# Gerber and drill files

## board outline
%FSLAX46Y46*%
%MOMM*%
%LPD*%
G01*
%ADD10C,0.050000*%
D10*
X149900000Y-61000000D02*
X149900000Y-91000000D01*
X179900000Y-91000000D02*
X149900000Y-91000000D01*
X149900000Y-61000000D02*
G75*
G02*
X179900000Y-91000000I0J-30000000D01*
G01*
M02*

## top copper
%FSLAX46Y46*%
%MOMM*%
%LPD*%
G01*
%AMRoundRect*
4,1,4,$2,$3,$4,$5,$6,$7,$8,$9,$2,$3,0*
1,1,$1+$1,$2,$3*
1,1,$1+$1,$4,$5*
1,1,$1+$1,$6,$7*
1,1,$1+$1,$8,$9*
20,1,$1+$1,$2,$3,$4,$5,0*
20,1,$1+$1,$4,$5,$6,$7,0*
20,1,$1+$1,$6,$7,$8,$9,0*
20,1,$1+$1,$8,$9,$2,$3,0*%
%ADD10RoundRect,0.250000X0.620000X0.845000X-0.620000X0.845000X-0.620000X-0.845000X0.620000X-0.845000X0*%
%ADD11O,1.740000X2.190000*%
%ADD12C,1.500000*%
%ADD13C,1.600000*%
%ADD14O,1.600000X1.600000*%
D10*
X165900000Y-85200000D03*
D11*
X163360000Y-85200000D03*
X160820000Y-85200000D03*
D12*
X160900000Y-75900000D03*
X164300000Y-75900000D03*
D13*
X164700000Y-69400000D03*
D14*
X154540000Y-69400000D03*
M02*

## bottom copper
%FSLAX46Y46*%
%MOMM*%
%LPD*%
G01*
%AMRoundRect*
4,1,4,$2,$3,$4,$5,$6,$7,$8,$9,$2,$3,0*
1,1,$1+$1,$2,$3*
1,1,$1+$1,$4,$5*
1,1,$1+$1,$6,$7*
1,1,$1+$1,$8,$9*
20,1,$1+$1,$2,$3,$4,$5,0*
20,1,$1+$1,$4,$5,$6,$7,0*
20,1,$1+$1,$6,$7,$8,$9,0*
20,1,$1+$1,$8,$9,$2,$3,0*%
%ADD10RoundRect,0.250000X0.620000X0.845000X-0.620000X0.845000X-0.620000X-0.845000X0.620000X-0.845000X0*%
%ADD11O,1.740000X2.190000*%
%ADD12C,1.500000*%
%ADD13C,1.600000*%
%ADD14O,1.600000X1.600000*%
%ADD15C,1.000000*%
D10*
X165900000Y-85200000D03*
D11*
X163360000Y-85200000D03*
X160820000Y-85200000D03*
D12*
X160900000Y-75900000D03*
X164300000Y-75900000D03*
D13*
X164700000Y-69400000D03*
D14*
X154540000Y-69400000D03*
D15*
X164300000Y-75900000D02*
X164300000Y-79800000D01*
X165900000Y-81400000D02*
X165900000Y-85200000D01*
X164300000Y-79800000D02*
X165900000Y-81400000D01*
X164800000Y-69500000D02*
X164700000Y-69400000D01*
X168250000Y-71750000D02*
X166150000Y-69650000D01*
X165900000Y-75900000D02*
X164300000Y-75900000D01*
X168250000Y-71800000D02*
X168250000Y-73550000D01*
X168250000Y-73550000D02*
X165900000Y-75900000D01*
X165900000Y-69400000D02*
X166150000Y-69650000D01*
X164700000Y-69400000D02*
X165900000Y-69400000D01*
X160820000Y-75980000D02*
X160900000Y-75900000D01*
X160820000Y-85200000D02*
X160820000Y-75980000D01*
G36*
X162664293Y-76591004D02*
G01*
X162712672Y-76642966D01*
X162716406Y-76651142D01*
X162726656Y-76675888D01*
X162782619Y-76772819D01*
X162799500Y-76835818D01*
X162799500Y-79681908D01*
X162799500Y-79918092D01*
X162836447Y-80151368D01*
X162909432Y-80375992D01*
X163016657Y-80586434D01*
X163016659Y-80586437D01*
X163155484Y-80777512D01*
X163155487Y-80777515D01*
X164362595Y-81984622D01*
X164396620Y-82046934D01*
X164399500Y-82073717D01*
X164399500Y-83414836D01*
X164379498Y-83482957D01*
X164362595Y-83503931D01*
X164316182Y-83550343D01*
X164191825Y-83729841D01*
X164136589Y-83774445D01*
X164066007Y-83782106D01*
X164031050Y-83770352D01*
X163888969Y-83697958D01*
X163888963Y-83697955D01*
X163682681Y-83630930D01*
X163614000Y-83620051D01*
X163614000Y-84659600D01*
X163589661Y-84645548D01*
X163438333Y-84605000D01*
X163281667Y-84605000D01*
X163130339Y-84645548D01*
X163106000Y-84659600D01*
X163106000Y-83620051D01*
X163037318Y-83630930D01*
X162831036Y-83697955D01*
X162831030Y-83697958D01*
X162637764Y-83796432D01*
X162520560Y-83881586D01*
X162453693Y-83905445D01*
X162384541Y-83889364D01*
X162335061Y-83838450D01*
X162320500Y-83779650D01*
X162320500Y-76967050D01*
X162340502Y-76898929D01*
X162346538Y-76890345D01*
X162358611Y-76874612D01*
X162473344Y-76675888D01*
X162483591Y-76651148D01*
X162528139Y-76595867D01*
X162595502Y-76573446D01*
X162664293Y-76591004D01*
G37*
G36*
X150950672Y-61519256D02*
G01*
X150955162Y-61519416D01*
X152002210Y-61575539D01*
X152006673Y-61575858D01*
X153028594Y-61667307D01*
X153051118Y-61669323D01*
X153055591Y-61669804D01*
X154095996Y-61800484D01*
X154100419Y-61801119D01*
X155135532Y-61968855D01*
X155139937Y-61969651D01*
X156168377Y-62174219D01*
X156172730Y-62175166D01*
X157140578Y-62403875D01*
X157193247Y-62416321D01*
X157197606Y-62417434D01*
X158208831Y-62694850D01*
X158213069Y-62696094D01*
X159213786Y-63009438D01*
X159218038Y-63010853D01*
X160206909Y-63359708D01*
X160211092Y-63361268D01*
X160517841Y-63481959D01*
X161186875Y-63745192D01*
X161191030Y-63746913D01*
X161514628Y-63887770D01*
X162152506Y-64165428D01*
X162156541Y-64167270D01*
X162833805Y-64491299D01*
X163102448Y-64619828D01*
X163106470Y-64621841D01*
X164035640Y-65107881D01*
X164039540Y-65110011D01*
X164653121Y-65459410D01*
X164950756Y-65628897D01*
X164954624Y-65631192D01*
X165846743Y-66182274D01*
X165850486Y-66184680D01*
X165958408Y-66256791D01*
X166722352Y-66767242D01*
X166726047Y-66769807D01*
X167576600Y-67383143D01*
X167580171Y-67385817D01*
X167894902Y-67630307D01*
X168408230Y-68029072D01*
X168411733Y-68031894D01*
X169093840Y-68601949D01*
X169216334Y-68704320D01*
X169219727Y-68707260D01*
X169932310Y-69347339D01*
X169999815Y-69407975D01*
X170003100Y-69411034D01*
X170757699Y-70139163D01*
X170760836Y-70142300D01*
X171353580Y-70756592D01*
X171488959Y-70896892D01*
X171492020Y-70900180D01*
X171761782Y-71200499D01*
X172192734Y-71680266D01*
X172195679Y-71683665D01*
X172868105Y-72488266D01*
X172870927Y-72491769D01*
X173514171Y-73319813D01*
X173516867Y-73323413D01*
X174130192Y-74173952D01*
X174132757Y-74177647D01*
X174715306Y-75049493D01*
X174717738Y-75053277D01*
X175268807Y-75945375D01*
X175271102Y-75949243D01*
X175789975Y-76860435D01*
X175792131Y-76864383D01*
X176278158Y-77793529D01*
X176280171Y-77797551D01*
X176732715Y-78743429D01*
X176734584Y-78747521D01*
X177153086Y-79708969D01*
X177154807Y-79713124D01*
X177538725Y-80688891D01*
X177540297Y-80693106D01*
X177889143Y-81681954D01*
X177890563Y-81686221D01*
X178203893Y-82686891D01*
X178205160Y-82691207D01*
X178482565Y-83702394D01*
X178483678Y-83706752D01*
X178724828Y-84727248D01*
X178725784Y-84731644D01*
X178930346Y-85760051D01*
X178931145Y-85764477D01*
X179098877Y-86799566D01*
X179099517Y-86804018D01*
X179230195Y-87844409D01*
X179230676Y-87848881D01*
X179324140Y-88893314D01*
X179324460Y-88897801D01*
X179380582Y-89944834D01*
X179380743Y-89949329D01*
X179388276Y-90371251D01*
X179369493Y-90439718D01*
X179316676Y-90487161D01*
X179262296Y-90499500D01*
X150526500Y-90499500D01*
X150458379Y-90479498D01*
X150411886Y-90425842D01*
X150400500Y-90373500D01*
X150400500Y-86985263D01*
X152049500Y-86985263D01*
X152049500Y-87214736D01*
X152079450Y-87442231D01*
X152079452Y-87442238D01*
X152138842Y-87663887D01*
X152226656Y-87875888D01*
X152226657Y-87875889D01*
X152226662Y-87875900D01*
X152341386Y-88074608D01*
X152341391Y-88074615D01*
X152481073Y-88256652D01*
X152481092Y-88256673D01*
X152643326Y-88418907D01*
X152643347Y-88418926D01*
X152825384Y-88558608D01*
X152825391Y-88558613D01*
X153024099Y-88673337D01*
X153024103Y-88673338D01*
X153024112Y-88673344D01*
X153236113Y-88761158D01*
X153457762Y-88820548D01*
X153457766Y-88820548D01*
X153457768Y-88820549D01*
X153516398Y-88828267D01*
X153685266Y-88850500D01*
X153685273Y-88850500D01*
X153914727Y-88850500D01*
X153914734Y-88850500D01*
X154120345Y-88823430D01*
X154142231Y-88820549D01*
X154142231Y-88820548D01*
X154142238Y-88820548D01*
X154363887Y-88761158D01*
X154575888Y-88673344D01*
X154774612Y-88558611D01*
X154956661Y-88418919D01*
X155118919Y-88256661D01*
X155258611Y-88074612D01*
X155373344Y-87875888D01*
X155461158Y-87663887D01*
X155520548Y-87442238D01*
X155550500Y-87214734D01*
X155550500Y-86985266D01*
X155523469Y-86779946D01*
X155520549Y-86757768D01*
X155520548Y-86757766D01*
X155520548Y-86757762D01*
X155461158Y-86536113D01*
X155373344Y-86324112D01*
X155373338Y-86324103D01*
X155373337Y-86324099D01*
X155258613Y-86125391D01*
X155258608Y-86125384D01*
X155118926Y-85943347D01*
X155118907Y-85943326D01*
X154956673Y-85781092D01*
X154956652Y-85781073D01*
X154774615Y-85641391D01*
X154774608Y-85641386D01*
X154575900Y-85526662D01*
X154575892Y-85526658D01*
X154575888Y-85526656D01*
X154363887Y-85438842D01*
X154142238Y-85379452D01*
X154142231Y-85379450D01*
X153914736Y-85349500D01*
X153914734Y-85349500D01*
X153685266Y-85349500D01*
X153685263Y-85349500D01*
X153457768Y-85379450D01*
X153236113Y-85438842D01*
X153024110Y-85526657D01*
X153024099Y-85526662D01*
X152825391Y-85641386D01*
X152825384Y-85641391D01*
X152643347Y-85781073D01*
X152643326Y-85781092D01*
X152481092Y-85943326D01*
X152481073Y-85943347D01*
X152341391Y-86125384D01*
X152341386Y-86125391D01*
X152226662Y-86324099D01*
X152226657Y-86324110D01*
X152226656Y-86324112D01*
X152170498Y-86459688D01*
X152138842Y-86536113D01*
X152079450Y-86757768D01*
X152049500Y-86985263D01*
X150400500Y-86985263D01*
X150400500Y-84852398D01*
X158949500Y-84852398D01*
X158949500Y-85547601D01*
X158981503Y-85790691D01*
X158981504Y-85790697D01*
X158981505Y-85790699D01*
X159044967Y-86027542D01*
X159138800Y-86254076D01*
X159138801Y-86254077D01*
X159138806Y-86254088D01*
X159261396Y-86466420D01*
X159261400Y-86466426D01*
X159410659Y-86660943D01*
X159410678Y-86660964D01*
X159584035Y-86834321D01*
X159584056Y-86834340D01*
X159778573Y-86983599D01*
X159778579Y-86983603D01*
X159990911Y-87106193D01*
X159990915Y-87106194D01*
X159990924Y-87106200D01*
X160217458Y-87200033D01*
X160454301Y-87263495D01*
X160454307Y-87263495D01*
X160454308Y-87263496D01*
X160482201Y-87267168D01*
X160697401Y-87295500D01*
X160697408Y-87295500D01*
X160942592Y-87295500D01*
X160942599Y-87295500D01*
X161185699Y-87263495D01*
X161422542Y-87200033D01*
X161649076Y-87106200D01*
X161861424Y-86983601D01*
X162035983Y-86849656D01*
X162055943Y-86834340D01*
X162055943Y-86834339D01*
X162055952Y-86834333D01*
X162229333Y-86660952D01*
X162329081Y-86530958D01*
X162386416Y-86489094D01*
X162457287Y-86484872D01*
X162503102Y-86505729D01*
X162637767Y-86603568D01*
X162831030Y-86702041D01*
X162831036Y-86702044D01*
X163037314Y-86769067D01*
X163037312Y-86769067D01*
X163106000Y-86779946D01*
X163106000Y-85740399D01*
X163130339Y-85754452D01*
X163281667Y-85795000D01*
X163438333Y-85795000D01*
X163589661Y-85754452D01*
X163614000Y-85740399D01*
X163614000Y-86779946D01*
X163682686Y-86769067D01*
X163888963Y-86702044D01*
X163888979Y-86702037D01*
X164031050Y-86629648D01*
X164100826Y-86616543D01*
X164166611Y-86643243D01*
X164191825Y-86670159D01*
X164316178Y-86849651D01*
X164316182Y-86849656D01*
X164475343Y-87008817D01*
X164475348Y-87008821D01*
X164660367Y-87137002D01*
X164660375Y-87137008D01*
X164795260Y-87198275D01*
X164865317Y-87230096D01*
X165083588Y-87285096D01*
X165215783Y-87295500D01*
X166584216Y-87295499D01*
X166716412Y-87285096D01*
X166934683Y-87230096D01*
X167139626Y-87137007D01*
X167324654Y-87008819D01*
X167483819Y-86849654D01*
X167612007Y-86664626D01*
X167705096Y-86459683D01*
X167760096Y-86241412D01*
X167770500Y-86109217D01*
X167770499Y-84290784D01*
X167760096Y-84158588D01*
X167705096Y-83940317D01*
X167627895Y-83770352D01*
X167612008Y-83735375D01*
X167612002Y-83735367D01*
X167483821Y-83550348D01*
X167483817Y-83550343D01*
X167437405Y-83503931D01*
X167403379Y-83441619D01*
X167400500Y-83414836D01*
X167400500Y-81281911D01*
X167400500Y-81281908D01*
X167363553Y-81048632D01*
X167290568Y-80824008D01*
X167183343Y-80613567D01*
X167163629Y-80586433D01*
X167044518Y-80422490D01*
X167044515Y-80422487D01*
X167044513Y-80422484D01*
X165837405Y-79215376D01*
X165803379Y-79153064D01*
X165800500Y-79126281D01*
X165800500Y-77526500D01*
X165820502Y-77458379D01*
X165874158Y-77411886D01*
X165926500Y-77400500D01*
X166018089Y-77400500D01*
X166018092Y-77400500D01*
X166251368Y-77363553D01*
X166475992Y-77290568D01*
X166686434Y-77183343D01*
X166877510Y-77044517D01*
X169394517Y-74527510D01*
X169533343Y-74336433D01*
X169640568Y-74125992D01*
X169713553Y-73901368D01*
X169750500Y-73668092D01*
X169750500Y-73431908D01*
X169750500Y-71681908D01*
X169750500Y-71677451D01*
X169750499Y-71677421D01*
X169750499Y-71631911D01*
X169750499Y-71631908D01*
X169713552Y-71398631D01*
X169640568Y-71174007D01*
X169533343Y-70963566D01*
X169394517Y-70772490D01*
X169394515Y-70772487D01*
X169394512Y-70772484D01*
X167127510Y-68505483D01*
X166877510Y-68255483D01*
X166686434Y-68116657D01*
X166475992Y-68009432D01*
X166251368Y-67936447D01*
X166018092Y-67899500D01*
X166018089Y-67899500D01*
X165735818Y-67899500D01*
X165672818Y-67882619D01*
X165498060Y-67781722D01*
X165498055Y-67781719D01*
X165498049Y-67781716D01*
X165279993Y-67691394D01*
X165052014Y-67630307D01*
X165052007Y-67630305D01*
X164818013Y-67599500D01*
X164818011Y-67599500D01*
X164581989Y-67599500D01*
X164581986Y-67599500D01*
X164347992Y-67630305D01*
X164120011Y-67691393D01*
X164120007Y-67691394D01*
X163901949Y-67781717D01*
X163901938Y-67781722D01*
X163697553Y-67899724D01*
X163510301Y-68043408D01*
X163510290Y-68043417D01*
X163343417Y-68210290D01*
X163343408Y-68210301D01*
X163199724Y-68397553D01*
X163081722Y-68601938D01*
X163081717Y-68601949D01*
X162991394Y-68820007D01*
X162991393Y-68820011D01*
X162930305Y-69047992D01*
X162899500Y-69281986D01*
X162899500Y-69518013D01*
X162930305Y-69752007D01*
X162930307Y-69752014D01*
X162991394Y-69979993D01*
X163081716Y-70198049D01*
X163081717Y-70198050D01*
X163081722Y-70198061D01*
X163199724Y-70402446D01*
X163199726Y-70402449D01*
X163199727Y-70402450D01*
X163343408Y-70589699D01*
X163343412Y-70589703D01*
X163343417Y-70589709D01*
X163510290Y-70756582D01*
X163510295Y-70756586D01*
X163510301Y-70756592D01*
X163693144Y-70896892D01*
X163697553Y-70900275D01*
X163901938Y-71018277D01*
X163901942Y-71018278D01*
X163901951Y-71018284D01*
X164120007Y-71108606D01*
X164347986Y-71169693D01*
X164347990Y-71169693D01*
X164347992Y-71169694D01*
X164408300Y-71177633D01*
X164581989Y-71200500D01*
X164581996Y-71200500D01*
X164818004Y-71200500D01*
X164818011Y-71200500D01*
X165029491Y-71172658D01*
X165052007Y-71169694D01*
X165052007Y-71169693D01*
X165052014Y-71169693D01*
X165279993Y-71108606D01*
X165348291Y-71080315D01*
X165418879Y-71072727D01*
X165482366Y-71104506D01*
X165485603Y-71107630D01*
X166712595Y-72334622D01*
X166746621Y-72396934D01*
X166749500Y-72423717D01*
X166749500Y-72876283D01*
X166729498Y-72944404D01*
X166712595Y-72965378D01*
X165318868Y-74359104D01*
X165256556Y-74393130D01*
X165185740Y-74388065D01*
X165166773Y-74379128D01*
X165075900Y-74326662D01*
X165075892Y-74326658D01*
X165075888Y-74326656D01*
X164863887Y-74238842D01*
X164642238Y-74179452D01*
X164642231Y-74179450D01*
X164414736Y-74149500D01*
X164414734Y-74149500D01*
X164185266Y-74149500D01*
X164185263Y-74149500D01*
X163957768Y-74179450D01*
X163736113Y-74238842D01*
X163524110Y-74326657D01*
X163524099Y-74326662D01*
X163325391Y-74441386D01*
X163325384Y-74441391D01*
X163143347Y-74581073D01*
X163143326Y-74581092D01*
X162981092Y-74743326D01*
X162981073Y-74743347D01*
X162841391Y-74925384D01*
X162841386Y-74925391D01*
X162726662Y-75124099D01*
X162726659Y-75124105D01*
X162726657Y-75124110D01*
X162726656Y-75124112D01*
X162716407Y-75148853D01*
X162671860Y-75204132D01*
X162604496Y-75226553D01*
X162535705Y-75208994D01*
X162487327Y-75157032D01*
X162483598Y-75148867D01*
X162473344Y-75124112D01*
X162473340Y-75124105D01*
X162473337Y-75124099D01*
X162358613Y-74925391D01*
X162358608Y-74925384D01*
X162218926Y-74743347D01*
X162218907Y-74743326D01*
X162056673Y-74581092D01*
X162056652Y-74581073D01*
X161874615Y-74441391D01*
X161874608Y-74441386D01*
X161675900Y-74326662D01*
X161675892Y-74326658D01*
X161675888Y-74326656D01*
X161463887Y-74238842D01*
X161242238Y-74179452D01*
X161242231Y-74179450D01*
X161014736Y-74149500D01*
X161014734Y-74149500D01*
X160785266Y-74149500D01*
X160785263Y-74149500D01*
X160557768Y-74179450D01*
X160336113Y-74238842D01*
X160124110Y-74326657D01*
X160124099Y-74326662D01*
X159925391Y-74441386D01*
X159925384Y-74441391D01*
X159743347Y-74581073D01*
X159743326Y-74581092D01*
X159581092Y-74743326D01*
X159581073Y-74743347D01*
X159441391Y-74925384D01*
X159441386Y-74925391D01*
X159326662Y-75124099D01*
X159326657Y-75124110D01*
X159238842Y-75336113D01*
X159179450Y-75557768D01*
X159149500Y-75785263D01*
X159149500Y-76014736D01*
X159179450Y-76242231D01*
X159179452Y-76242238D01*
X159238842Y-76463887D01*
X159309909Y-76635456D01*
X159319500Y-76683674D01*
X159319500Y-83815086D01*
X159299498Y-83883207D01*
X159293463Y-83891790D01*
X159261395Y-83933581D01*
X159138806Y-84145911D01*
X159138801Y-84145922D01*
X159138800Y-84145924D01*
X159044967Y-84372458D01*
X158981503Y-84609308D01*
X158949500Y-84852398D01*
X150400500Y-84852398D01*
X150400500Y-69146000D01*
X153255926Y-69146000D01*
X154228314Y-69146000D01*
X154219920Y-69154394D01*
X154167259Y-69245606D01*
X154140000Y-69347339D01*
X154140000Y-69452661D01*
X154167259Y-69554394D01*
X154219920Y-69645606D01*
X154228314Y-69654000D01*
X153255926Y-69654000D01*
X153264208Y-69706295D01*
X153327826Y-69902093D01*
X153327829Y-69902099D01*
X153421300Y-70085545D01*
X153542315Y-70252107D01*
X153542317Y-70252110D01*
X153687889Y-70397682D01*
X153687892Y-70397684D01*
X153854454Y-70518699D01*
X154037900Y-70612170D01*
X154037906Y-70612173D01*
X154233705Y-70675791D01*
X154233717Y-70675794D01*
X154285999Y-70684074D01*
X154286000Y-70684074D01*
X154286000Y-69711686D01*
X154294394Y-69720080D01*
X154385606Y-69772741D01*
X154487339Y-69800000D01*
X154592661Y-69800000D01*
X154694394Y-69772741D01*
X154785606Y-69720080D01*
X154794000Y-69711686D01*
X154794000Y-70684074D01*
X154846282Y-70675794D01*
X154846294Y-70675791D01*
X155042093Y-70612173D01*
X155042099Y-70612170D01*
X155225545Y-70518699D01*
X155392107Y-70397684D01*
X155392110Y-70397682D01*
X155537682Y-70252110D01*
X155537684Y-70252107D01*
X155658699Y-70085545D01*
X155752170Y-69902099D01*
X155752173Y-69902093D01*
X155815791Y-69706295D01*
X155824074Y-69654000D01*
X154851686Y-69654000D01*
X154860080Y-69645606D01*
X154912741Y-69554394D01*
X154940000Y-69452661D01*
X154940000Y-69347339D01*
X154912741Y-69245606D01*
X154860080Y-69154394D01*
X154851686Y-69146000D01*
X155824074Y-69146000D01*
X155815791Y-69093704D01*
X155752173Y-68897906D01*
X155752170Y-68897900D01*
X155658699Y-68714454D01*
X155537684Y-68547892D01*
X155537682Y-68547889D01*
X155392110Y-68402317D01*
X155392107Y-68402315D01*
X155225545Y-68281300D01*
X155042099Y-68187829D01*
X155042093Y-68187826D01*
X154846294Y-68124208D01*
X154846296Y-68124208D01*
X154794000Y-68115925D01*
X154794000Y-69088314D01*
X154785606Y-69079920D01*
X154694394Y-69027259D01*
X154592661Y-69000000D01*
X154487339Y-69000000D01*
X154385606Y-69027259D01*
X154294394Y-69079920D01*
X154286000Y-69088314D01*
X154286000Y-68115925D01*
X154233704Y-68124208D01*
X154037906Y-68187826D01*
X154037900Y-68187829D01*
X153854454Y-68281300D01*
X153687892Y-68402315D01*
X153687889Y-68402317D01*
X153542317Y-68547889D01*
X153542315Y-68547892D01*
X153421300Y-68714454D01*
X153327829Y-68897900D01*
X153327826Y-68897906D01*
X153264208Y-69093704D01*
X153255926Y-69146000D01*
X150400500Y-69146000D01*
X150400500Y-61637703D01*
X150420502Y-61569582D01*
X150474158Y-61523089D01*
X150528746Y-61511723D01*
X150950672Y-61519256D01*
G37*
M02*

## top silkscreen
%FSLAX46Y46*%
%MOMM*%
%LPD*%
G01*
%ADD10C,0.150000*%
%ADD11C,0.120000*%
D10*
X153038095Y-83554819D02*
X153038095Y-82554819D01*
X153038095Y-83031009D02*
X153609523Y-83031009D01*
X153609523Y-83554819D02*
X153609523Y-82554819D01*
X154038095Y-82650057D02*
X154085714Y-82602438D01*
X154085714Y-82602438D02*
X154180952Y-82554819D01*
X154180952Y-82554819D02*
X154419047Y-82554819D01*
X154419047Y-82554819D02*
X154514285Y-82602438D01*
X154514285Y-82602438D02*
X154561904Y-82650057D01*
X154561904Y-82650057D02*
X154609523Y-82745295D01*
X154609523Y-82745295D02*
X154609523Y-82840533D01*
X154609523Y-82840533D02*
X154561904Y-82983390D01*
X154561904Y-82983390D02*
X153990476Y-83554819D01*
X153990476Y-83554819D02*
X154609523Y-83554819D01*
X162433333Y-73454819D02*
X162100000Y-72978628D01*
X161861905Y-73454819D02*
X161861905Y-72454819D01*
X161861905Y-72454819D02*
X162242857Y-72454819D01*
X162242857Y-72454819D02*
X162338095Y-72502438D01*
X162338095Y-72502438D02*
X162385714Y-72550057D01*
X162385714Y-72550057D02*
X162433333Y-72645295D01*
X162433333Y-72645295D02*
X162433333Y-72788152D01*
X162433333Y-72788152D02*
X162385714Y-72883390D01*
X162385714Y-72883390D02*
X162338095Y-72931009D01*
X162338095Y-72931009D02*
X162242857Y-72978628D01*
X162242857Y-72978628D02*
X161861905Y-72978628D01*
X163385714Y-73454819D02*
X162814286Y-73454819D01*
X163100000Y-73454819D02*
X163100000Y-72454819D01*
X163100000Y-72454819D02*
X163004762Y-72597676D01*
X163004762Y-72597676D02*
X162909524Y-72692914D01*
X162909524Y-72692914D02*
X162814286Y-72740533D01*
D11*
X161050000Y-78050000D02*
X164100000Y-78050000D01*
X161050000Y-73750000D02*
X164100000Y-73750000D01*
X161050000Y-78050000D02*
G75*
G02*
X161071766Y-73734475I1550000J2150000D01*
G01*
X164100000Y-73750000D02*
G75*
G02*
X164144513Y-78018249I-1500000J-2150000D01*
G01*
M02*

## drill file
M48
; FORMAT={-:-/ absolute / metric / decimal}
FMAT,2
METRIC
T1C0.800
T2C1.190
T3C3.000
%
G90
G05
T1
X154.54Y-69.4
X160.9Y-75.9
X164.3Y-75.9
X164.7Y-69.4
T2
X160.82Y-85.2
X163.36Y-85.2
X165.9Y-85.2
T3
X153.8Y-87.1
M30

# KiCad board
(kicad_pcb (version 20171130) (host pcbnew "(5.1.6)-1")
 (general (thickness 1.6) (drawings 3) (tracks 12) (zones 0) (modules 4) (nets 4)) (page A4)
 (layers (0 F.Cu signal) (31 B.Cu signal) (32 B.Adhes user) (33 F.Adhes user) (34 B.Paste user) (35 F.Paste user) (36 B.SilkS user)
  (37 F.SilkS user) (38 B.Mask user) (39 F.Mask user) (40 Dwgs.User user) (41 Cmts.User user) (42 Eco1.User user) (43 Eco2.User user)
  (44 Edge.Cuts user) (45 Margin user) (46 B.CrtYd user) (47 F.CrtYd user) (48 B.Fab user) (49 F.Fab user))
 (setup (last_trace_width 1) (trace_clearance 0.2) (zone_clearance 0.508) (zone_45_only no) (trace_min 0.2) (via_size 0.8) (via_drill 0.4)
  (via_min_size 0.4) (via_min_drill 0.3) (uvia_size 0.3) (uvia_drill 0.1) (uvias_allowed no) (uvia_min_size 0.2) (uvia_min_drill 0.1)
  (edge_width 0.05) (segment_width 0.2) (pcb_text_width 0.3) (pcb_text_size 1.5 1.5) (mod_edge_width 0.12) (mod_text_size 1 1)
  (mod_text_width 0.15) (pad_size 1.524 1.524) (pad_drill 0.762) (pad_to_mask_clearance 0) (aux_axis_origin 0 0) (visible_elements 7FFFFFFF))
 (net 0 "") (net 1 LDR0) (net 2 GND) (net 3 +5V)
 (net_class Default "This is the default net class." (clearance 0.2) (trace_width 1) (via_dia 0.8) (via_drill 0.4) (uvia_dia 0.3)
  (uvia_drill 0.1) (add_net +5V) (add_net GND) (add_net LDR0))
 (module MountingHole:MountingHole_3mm (layer F.Cu) (at 153.8 87.1)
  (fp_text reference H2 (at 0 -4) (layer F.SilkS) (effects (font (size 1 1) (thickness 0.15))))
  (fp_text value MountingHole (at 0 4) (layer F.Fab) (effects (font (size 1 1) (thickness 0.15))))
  (pad 1 np_thru_hole circle (at 0 0) (size 3 3) (drill 3) (layers *.Cu *.Mask)))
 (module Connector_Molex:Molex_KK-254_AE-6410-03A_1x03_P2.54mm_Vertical (layer B.Cu) (at 165.9 85.2 180)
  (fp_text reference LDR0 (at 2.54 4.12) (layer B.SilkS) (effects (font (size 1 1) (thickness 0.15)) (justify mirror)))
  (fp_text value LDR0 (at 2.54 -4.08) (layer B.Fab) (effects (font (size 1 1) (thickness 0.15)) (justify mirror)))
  (pad 1 thru_hole roundrect (at 0 0 180) (size 1.74 2.19) (drill 1.19) (layers *.Cu *.Mask) (roundrect_rratio 0.143678) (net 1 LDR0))
  (pad 2 thru_hole oval (at 2.54 0 180) (size 1.74 2.19) (drill 1.19) (layers *.Cu *.Mask) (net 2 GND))
  (pad 3 thru_hole oval (at 5.08 0 180) (size 1.74 2.19) (drill 1.19) (layers *.Cu *.Mask) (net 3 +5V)))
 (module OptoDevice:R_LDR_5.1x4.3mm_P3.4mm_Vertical (layer F.Cu) (at 160.9 75.9)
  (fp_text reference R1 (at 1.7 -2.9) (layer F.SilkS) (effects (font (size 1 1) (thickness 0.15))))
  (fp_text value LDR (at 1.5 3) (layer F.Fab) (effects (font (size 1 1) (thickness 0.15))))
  (fp_line (start 0.15 2.15) (end 3.2 2.15) (layer F.SilkS) (width 0.12))
  (fp_line (start 0.15 -2.15) (end 3.2 -2.15) (layer F.SilkS) (width 0.12))
  (fp_arc (start 1.7 0) (end 0.15 2.15) (angle 109) (layer F.SilkS) (width 0.12))
  (fp_arc (start 1.7 0) (end 3.2 -2.15) (angle 109) (layer F.SilkS) (width 0.12))
  (pad 1 thru_hole circle (at 0 0) (size 1.5 1.5) (drill 0.8) (layers *.Cu *.Mask) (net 3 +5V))
  (pad 2 thru_hole circle (at 3.4 0) (size 1.5 1.5) (drill 0.8) (layers *.Cu *.Mask) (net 1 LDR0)))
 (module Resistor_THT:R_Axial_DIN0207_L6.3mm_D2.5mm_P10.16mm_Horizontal (layer B.Cu) (at 164.7 69.4 180)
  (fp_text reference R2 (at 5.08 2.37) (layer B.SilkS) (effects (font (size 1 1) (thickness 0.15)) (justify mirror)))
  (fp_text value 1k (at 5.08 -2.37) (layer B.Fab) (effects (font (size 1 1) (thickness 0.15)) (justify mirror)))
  (pad 1 thru_hole circle (at 0 0 180) (size 1.6 1.6) (drill 0.8) (layers *.Cu *.Mask) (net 1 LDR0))
  (pad 2 thru_hole oval (at 10.16 0 180) (size 1.6 1.6) (drill 0.8) (layers *.Cu *.Mask) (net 2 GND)))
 (gr_line (start 149.9 61) (end 149.9 91) (layer Edge.Cuts) (width 0.05))
 (gr_line (start 179.9 91) (end 149.9 91) (layer Edge.Cuts) (width 0.05))
 (gr_arc (start 149.9 91) (end 179.9 91) (angle -90) (layer Edge.Cuts) (width 0.05))
 (segment (start 164.3 75.9) (end 164.3 79.8) (width 1) (layer B.Cu) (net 1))
 (segment (start 165.9 81.4) (end 165.9 85.2) (width 1) (layer B.Cu) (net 1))
 (segment (start 164.3 79.8) (end 165.9 81.4) (width 1) (layer B.Cu) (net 1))
 (segment (start 164.8 69.5) (end 164.7 69.4) (width 1) (layer B.Cu) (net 1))
 (segment (start 168.25 71.75) (end 166.15 69.65) (width 1) (layer B.Cu) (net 1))
 (segment (start 165.9 75.9) (end 164.3 75.9) (width 1) (layer B.Cu) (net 1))
 (segment (start 168.25 71.8) (end 168.25 73.55) (width 1) (layer B.Cu) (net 1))
 (segment (start 168.25 73.55) (end 165.9 75.9) (width 1) (layer B.Cu) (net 1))
 (segment (start 165.9 69.4) (end 166.15 69.65) (width 1) (layer B.Cu) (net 1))
 (segment (start 164.7 69.4) (end 165.9 69.4) (width 1) (layer B.Cu) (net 1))
 (segment (start 160.82 75.98) (end 160.9 75.9) (width 1) (layer B.Cu) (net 3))
 (segment (start 160.82 85.2) (end 160.82 75.98) (width 1) (layer B.Cu) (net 3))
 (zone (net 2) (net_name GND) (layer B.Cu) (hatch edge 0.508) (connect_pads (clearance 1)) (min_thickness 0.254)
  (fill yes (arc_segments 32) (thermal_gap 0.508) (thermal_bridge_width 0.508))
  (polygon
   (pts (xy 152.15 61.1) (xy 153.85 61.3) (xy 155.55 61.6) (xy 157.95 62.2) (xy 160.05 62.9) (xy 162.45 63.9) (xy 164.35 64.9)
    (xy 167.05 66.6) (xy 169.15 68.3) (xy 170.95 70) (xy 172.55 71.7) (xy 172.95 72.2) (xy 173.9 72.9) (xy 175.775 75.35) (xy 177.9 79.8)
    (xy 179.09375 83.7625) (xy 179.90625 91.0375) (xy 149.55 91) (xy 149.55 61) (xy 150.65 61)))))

